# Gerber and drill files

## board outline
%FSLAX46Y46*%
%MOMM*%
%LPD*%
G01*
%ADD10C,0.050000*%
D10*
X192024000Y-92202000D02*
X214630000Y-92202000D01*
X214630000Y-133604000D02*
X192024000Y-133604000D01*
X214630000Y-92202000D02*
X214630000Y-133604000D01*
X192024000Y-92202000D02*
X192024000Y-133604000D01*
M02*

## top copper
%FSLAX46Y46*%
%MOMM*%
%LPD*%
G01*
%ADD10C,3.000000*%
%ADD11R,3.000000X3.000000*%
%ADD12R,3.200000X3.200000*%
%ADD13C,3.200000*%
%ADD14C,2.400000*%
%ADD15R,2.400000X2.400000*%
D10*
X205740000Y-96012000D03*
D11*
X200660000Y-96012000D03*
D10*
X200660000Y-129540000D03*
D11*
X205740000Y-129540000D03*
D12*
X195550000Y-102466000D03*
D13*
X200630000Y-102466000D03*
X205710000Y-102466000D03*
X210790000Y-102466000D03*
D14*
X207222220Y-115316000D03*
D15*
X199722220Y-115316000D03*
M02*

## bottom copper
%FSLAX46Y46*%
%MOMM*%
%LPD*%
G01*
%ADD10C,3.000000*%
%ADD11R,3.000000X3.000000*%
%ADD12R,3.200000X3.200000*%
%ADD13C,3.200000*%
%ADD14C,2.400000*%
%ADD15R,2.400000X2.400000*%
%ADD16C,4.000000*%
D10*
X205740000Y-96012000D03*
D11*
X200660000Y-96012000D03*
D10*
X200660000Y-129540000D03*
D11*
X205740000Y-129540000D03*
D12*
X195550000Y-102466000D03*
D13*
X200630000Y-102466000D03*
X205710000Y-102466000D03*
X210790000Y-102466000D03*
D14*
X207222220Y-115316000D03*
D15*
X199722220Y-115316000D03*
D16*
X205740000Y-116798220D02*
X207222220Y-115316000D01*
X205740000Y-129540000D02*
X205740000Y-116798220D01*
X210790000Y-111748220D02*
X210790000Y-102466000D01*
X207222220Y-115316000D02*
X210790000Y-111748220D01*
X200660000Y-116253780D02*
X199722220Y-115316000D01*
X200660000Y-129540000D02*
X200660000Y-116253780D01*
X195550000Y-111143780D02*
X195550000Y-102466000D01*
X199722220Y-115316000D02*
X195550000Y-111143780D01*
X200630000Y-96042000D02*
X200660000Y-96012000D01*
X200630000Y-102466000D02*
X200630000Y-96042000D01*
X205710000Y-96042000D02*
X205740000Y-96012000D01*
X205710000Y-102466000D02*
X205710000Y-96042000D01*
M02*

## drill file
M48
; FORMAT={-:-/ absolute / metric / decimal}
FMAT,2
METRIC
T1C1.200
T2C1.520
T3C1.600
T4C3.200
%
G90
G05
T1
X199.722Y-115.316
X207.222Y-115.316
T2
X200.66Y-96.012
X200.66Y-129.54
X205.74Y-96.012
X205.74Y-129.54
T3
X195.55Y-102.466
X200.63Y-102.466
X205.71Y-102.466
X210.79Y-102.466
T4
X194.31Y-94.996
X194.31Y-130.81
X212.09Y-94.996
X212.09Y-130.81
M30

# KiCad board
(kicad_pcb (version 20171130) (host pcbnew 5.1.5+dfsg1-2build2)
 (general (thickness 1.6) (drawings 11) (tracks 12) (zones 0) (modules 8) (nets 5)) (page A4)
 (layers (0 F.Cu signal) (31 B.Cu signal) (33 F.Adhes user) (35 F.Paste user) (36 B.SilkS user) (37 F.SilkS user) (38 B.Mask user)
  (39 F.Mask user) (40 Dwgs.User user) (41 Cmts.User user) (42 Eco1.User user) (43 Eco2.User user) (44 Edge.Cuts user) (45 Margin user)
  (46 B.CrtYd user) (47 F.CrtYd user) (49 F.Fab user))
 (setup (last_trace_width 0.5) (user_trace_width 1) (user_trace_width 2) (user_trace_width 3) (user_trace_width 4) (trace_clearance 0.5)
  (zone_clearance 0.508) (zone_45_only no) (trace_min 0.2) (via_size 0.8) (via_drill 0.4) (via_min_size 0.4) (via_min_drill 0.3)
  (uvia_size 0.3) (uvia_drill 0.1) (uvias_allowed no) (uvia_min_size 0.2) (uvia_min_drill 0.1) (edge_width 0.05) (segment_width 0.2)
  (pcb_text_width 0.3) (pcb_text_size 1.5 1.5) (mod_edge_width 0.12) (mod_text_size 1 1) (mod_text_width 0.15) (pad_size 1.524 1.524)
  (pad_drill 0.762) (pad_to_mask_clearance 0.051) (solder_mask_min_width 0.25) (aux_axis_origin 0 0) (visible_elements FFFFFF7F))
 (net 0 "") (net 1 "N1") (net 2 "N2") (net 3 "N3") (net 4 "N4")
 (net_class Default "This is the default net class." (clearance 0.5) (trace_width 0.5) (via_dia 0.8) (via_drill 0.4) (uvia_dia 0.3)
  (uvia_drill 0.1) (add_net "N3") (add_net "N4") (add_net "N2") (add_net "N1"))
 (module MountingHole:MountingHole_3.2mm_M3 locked (layer F.Cu) (at 194.31 130.81)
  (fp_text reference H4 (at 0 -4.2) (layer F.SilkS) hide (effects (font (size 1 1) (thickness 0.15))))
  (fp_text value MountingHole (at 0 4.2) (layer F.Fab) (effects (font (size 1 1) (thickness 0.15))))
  (pad 1 np_thru_hole circle (at 0 0) (size 3.2 3.2) (drill 3.2) (layers *.Cu *.Mask)))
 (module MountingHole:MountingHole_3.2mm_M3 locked (layer F.Cu) (at 212.09 130.81)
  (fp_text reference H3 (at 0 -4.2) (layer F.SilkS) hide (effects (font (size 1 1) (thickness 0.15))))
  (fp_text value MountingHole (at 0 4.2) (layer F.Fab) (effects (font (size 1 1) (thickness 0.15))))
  (pad 1 np_thru_hole circle (at 0 0) (size 3.2 3.2) (drill 3.2) (layers *.Cu *.Mask)))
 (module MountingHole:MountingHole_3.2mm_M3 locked (layer F.Cu) (at 194.31 94.996)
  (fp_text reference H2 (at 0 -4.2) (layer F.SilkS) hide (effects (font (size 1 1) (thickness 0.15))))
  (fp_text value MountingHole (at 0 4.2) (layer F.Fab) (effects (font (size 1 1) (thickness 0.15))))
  (pad 1 np_thru_hole circle (at 0 0) (size 3.2 3.2) (drill 3.2) (layers *.Cu *.Mask)))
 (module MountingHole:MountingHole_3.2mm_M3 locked (layer F.Cu) (at 212.09 94.996)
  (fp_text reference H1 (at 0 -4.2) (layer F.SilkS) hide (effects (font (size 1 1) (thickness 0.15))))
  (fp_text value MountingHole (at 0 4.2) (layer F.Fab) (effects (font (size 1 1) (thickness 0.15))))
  (pad 1 np_thru_hole circle (at 0 0) (size 3.2 3.2) (drill 3.2) (layers *.Cu *.Mask)))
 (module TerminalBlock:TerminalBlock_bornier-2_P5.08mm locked (layer F.Cu) (at 200.66 96.012)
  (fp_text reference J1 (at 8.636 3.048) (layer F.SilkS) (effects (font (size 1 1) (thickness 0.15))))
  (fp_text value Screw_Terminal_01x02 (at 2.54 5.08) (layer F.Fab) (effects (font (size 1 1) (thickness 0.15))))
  (pad 2 thru_hole circle (at 5.08 0) (size 3 3) (drill 1.52) (layers *.Cu *.Mask) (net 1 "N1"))
  (pad 1 thru_hole rect (at 0 0) (size 3 3) (drill 1.52) (layers *.Cu *.Mask) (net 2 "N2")))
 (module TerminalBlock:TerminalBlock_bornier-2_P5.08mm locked (layer F.Cu) (at 205.74 129.54 180)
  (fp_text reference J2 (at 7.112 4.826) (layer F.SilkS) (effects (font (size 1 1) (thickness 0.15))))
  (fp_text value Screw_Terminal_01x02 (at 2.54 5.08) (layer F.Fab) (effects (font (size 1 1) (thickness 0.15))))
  (pad 2 thru_hole circle (at 5.08 0 180) (size 3 3) (drill 1.52) (layers *.Cu *.Mask) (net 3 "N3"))
  (pad 1 thru_hole rect (at 0 0 180) (size 3 3) (drill 1.52) (layers *.Cu *.Mask) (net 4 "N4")))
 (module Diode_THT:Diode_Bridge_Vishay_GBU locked (layer F.Cu) (at 195.55 102.466)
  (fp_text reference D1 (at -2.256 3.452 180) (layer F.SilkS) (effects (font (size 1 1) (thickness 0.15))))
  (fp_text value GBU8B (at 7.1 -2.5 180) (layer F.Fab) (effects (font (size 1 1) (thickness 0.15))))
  (pad 1 thru_hole rect (at 0 0) (size 3.2 3.2) (drill 1.6) (layers *.Cu *.Mask) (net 3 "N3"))
  (pad 2 thru_hole circle (at 5.08 0) (size 3.2 3.2) (drill 1.6) (layers *.Cu *.Mask) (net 2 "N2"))
  (pad 3 thru_hole circle (at 10.16 0) (size 3.2 3.2) (drill 1.6) (layers *.Cu *.Mask) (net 1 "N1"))
  (pad 4 thru_hole circle (at 15.24 0) (size 3.2 3.2) (drill 1.6) (layers *.Cu *.Mask) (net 4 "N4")))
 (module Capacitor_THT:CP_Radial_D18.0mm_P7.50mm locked (layer F.Cu) (at 199.72222 115.316)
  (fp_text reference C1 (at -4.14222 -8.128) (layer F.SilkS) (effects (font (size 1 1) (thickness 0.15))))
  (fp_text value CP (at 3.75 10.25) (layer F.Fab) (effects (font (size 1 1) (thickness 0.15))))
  (pad 2 thru_hole circle (at 7.5 0) (size 2.4 2.4) (drill 1.2) (layers *.Cu *.Mask) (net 4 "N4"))
  (pad 1 thru_hole rect (at 0 0) (size 2.4 2.4) (drill 1.2) (layers *.Cu *.Mask) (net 3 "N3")))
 (gr_line (start 192.024 92.202) (end 214.63 92.202) (layer Edge.Cuts) (width 0.05))
 (gr_line (start 214.63 133.604) (end 192.024 133.604) (layer Edge.Cuts) (width 0.05))
 (gr_line (start 214.63 92.202) (end 214.63 133.604) (layer Edge.Cuts) (width 0.05))
 (gr_line (start 192.024 92.202) (end 192.024 133.604) (layer Edge.Cuts) (width 0.05))
 (segment (start 205.74 116.79822) (end 207.22222 115.316) (width 4) (layer B.Cu) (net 4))
 (segment (start 205.74 129.54) (end 205.74 116.79822) (width 4) (layer B.Cu) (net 4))
 (segment (start 210.79 111.74822) (end 210.79 102.466) (width 4) (layer B.Cu) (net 4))
 (segment (start 207.22222 115.316) (end 210.79 111.74822) (width 4) (layer B.Cu) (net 4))
 (segment (start 200.66 116.25378) (end 199.72222 115.316) (width 4) (layer B.Cu) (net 3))
 (segment (start 200.66 129.54) (end 200.66 116.25378) (width 4) (layer B.Cu) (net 3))
 (segment (start 195.55 111.14378) (end 195.55 102.466) (width 4) (layer B.Cu) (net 3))
 (segment (start 199.72222 115.316) (end 195.55 111.14378) (width 4) (layer B.Cu) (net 3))
 (segment (start 200.63 96.042) (end 200.66 96.012) (width 4) (layer B.Cu) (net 2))
 (segment (start 200.63 102.466) (end 200.63 96.042) (width 4) (layer B.Cu) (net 2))
 (segment (start 205.71 96.042) (end 205.74 96.012) (width 4) (layer B.Cu) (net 1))
 (segment (start 205.71 102.466) (end 205.71 96.042) (width 4) (layer B.Cu) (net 1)))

